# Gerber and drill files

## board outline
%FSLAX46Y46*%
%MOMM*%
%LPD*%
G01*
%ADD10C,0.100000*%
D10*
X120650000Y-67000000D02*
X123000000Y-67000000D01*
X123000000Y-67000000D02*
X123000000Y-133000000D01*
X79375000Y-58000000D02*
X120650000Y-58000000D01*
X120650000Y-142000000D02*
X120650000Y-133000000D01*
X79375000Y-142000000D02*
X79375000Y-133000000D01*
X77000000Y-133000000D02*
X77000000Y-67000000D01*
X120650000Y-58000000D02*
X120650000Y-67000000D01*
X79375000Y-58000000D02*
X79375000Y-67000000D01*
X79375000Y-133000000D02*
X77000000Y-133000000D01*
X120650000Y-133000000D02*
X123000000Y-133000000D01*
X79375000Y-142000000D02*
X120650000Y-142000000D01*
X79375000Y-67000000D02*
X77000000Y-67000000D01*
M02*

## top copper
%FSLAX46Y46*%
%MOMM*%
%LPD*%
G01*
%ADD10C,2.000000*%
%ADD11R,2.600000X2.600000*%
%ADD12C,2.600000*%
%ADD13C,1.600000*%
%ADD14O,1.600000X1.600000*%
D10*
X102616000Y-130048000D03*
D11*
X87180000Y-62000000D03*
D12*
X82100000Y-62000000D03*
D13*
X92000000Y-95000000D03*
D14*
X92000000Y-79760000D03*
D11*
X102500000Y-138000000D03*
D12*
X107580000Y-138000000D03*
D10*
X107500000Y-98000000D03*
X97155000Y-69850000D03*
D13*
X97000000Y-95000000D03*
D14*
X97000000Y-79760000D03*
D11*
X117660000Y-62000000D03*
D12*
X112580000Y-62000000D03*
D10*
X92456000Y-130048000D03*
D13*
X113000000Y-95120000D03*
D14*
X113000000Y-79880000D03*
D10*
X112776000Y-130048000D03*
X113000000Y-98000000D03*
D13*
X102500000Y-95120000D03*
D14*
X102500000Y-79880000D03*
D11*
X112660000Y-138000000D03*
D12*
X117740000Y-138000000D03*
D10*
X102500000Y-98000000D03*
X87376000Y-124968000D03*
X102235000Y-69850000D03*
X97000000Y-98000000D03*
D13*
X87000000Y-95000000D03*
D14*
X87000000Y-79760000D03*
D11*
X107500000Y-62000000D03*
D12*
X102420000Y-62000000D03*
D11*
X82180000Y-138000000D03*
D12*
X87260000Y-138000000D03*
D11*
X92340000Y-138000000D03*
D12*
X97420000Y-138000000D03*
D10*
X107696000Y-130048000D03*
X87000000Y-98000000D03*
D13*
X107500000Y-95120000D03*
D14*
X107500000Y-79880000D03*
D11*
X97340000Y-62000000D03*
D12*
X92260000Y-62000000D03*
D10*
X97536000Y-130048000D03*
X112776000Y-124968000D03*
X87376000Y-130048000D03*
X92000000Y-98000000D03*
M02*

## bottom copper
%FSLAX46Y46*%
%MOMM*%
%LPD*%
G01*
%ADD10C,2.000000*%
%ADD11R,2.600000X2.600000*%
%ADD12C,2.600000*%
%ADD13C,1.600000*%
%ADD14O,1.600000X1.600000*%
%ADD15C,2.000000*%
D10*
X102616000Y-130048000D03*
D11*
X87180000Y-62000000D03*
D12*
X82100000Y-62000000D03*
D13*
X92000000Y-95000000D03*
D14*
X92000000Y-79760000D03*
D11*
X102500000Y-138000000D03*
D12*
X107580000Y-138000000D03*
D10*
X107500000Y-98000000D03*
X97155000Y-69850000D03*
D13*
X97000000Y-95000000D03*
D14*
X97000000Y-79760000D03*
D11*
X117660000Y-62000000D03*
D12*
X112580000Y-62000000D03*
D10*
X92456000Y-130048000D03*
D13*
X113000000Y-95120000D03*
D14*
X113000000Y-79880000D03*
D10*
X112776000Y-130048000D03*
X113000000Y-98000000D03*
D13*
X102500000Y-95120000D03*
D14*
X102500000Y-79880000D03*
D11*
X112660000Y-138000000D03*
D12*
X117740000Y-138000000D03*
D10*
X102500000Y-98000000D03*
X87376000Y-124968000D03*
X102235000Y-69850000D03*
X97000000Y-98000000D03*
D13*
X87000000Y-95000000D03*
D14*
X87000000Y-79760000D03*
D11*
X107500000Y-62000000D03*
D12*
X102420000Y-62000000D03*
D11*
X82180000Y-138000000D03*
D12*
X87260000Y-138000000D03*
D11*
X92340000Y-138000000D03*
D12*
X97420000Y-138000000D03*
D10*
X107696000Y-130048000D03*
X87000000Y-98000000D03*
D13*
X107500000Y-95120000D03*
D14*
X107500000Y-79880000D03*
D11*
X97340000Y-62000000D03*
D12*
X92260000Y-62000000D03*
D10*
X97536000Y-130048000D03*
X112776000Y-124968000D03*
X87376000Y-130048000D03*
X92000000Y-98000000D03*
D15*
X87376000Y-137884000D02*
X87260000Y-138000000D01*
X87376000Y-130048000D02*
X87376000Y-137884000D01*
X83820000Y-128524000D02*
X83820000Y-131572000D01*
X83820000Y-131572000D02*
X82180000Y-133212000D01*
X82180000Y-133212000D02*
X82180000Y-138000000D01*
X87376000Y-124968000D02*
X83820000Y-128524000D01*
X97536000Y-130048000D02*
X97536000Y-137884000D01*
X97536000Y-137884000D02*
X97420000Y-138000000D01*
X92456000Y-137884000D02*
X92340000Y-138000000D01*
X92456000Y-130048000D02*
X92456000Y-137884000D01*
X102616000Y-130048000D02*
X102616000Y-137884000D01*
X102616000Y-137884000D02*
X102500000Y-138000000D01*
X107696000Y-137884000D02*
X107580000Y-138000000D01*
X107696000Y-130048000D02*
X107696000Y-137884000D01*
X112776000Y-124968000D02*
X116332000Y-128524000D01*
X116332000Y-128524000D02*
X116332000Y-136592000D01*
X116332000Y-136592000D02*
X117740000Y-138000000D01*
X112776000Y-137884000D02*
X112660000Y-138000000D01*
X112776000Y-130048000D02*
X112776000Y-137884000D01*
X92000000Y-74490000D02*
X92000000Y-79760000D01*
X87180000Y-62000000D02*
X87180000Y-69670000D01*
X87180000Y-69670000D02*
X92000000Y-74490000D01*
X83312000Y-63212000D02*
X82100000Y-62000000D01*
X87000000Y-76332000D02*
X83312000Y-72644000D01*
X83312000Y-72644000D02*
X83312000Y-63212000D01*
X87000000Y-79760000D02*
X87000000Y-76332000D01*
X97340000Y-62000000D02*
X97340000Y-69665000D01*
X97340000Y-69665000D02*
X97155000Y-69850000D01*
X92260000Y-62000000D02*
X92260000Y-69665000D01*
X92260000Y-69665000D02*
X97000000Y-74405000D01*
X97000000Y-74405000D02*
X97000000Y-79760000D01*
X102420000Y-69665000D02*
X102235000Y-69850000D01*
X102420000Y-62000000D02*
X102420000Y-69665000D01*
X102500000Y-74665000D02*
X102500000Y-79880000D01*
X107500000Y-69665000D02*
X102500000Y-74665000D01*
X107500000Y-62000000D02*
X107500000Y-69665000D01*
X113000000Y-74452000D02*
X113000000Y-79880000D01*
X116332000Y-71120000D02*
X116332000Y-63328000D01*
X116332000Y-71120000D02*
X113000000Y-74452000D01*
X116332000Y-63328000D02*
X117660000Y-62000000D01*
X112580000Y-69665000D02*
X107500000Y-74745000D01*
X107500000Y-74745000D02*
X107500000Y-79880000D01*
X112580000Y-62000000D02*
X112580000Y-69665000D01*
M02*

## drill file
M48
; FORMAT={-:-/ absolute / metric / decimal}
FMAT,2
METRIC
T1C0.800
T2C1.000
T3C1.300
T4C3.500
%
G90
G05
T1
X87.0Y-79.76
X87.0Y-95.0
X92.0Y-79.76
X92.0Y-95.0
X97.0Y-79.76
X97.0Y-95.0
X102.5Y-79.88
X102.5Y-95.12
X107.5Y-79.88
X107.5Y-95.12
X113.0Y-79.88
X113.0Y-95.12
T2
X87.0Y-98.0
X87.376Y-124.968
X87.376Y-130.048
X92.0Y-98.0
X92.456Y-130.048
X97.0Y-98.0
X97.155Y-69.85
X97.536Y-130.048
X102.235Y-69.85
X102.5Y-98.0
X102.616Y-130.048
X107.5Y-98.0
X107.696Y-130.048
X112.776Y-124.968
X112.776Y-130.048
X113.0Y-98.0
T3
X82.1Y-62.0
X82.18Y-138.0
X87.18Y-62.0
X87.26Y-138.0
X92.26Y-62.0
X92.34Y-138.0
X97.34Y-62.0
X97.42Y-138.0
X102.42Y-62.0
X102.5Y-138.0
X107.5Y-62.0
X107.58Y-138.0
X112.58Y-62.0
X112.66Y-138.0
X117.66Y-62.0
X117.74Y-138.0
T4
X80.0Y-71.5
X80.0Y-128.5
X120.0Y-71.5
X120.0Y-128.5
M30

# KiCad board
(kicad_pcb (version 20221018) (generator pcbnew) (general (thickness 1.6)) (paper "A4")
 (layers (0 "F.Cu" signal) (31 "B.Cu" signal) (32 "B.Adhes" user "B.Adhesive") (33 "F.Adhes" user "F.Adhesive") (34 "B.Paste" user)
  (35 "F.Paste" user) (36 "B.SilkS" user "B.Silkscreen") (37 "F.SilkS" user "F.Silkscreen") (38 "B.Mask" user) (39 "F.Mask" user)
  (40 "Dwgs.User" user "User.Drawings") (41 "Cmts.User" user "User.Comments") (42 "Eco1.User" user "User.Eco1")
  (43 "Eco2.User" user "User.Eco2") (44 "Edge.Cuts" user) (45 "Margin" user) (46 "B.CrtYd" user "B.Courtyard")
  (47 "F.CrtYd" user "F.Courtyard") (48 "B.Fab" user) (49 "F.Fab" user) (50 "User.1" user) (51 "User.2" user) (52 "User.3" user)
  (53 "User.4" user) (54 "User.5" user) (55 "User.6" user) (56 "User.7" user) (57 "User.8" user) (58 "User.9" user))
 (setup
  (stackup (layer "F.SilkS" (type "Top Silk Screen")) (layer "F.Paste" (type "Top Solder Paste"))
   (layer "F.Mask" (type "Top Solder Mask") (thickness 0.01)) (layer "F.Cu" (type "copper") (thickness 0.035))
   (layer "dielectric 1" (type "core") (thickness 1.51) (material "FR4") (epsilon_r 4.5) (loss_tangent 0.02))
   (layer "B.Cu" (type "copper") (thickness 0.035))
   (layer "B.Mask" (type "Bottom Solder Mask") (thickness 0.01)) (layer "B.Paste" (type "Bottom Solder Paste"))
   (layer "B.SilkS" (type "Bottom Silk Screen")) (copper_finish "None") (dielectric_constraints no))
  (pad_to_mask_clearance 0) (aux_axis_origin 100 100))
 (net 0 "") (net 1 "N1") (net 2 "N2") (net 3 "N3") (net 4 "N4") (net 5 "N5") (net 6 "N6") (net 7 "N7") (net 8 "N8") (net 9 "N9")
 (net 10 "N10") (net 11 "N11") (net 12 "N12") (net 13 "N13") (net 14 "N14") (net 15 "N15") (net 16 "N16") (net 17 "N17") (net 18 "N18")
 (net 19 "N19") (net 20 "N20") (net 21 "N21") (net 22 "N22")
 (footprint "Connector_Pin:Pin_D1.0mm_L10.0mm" (layer "F.Cu") (at 102.616 130.048)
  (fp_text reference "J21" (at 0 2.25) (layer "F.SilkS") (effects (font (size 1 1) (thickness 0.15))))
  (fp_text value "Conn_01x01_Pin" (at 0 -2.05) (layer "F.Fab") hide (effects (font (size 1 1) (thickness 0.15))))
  (pad "1" thru_hole circle (at 0 0) (size 2 2) (drill 1) (layers "*.Cu" "*.Mask") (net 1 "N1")))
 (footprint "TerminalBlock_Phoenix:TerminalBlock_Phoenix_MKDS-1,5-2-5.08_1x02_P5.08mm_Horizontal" (layer "F.Cu") (at 87.18 62 180)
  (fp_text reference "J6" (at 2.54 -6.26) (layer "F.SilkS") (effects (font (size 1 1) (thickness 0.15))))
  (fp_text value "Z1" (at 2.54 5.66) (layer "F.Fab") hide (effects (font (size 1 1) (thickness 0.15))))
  (pad "1" thru_hole rect (at 0 0 180) (size 2.6 2.6) (drill 1.3) (layers "*.Cu" "*.Mask") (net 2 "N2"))
  (pad "2" thru_hole circle (at 5.08 0 180) (size 2.6 2.6) (drill 1.3) (layers "*.Cu" "*.Mask") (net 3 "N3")))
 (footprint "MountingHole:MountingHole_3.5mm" (layer "F.Cu") (at 80 71.5)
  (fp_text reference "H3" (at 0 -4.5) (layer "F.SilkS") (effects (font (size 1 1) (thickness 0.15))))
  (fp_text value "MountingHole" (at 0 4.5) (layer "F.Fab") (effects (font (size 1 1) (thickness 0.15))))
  (pad "" np_thru_hole circle (at 0 0) (size 3.5 3.5) (drill 3.5) (layers "*.Cu" "*.Mask")))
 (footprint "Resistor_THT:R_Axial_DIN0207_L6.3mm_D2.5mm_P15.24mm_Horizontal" (layer "F.Cu") (at 92 95 90)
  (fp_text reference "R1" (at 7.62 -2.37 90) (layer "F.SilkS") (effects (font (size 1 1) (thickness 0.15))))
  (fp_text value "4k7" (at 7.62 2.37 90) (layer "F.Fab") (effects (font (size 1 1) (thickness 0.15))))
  (pad "1" thru_hole circle (at 0 0 90) (size 1.6 1.6) (drill 0.8) (layers "*.Cu" "*.Mask") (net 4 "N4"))
  (pad "2" thru_hole oval (at 15.24 0 90) (size 1.6 1.6) (drill 0.8) (layers "*.Cu" "*.Mask") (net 2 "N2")))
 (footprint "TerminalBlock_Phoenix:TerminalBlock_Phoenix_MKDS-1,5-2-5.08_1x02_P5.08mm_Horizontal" (layer "F.Cu") (at 102.5 138)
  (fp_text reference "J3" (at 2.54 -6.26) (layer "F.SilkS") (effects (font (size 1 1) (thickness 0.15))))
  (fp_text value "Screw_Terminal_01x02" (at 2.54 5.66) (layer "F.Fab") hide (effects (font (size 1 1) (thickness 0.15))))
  (pad "1" thru_hole rect (at 0 0) (size 2.6 2.6) (drill 1.3) (layers "*.Cu" "*.Mask") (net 1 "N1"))
  (pad "2" thru_hole circle (at 5.08 0) (size 2.6 2.6) (drill 1.3) (layers "*.Cu" "*.Mask") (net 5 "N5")))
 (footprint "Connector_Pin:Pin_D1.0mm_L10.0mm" (layer "F.Cu") (at 107.5 98)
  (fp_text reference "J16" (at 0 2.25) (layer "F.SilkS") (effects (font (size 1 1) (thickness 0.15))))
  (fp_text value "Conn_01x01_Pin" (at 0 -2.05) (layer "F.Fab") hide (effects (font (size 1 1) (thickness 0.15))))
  (pad "1" thru_hole circle (at 0 0) (size 2 2) (drill 1) (layers "*.Cu" "*.Mask") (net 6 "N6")))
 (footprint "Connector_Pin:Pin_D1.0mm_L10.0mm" (layer "F.Cu") (at 97.155 69.85)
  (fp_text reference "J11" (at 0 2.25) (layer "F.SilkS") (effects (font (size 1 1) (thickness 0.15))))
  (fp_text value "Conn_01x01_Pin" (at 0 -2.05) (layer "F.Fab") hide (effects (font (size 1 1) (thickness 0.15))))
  (pad "1" thru_hole circle (at 0 0) (size 2 2) (drill 1) (layers "*.Cu" "*.Mask") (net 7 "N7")))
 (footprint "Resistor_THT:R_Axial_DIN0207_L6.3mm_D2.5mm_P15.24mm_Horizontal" (layer "F.Cu") (at 97 95 90)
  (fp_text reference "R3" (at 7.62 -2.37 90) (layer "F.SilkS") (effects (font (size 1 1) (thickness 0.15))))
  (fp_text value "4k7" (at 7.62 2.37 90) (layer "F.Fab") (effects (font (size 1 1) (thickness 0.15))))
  (pad "1" thru_hole circle (at 0 0 90) (size 1.6 1.6) (drill 0.8) (layers "*.Cu" "*.Mask") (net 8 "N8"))
  (pad "2" thru_hole oval (at 15.24 0 90) (size 1.6 1.6) (drill 0.8) (layers "*.Cu" "*.Mask") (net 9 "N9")))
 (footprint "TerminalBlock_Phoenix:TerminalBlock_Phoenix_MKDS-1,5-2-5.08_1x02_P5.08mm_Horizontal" (layer "F.Cu") (at 117.66 62 180)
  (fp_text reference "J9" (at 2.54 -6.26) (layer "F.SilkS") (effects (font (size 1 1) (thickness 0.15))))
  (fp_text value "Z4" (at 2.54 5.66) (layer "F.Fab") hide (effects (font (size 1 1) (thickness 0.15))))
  (pad "1" thru_hole rect (at 0 0 180) (size 2.6 2.6) (drill 1.3) (layers "*.Cu" "*.Mask") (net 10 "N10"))
  (pad "2" thru_hole circle (at 5.08 0 180) (size 2.6 2.6) (drill 1.3) (layers "*.Cu" "*.Mask") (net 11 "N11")))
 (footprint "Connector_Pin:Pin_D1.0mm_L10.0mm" (layer "F.Cu") (at 92.456 130.048)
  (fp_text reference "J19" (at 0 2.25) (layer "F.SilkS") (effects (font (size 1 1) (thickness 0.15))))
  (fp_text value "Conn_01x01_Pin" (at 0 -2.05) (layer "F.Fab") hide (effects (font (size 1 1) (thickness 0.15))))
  (pad "1" thru_hole circle (at 0 0) (size 2 2) (drill 1) (layers "*.Cu" "*.Mask") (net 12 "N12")))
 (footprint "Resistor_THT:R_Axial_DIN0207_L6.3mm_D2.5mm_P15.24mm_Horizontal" (layer "F.Cu") (at 113 95.12 90)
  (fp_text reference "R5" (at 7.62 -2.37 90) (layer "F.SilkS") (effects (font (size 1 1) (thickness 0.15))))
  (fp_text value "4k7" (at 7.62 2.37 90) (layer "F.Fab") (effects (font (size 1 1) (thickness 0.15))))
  (pad "1" thru_hole circle (at 0 0 90) (size 1.6 1.6) (drill 0.8) (layers "*.Cu" "*.Mask") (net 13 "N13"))
  (pad "2" thru_hole oval (at 15.24 0 90) (size 1.6 1.6) (drill 0.8) (layers "*.Cu" "*.Mask") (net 10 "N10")))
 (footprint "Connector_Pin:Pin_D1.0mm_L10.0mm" (layer "F.Cu") (at 112.776 130.048)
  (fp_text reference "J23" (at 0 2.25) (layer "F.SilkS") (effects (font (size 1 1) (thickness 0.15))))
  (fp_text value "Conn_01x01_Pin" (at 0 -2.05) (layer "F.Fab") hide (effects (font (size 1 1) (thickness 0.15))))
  (pad "1" thru_hole circle (at 0 0) (size 2 2) (drill 1) (layers "*.Cu" "*.Mask") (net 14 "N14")))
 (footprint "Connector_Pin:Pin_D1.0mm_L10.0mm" (layer "F.Cu") (at 113 98)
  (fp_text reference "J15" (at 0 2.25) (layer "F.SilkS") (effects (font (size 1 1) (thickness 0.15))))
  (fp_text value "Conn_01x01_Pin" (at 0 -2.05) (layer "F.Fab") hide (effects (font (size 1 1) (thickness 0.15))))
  (pad "1" thru_hole circle (at 0 0) (size 2 2) (drill 1) (layers "*.Cu" "*.Mask") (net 13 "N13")))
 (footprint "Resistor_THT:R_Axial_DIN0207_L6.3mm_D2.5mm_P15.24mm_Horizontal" (layer "F.Cu") (at 102.5 95.12 90)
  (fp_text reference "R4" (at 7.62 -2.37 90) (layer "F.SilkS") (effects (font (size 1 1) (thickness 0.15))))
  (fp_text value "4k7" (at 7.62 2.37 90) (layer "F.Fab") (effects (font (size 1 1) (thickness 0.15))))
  (pad "1" thru_hole circle (at 0 0 90) (size 1.6 1.6) (drill 0.8) (layers "*.Cu" "*.Mask") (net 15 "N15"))
  (pad "2" thru_hole oval (at 15.24 0 90) (size 1.6 1.6) (drill 0.8) (layers "*.Cu" "*.Mask") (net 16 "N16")))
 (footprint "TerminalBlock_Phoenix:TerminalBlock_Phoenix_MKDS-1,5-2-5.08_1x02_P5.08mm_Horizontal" (layer "F.Cu") (at 112.66 138)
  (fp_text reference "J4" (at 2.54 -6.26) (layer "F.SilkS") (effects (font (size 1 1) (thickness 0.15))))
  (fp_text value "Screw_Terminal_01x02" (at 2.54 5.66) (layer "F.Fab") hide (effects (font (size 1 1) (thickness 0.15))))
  (pad "1" thru_hole rect (at 0 0) (size 2.6 2.6) (drill 1.3) (layers "*.Cu" "*.Mask") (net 14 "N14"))
  (pad "2" thru_hole circle (at 5.08 0) (size 2.6 2.6) (drill 1.3) (layers "*.Cu" "*.Mask") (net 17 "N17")))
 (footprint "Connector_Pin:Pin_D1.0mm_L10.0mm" (layer "F.Cu") (at 102.5 98)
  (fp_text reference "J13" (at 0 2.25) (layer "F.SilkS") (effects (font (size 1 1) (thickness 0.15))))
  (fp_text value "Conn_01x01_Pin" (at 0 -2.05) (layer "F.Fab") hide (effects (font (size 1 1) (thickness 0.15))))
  (pad "1" thru_hole circle (at 0 0) (size 2 2) (drill 1) (layers "*.Cu" "*.Mask") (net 15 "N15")))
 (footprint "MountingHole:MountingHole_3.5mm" (layer "F.Cu") (at 120 128.5)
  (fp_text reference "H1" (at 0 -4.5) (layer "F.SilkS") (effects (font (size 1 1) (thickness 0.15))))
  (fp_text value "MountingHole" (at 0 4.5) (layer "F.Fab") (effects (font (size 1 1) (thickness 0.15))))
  (pad "" np_thru_hole circle (at 0 0) (size 3.5 3.5) (drill 3.5) (layers "*.Cu" "*.Mask")))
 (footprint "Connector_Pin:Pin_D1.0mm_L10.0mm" (layer "F.Cu") (at 87.376 124.968)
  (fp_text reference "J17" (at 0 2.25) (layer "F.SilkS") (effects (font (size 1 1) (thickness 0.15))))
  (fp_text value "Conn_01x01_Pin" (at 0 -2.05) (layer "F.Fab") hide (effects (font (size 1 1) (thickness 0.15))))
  (pad "1" thru_hole circle (at 0 0) (size 2 2) (drill 1) (layers "*.Cu" "*.Mask") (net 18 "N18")))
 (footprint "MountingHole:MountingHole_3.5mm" (layer "F.Cu") (at 80 128.5)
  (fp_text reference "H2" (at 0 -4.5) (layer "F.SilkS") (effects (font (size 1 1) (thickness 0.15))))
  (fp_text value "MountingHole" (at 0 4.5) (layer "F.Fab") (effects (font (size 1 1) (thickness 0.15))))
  (pad "" np_thru_hole circle (at 0 0) (size 3.5 3.5) (drill 3.5) (layers "*.Cu" "*.Mask")))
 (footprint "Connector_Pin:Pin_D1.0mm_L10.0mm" (layer "F.Cu") (at 102.235 69.85)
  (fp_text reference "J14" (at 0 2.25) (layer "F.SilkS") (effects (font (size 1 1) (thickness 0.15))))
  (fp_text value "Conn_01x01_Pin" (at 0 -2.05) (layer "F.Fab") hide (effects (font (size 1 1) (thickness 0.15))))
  (pad "1" thru_hole circle (at 0 0) (size 2 2) (drill 1) (layers "*.Cu" "*.Mask") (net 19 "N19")))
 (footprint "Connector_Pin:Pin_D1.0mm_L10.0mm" (layer "F.Cu") (at 97 98)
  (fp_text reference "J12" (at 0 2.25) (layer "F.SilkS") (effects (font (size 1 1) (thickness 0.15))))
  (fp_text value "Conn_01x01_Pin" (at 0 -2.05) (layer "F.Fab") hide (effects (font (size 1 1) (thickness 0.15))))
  (pad "1" thru_hole circle (at 0 0) (size 2 2) (drill 1) (layers "*.Cu" "*.Mask") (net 8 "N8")))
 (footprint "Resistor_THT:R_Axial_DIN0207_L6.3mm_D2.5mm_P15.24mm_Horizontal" (layer "F.Cu") (at 87 95 90)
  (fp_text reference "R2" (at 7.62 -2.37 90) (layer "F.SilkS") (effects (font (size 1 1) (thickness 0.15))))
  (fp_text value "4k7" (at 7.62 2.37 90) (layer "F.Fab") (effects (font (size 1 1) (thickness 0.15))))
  (pad "1" thru_hole circle (at 0 0 90) (size 1.6 1.6) (drill 0.8) (layers "*.Cu" "*.Mask") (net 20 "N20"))
  (pad "2" thru_hole oval (at 15.24 0 90) (size 1.6 1.6) (drill 0.8) (layers "*.Cu" "*.Mask") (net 3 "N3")))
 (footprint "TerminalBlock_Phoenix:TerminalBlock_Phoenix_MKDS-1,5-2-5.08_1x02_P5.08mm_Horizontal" (layer "F.Cu") (at 107.5 62 180)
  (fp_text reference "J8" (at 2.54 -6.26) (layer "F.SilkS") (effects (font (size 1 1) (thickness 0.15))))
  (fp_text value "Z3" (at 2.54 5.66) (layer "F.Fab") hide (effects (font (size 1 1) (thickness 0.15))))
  (pad "1" thru_hole rect (at 0 0 180) (size 2.6 2.6) (drill 1.3) (layers "*.Cu" "*.Mask") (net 16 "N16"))
  (pad "2" thru_hole circle (at 5.08 0 180) (size 2.6 2.6) (drill 1.3) (layers "*.Cu" "*.Mask") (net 19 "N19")))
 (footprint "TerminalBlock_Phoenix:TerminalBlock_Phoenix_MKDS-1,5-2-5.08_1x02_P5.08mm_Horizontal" (layer "F.Cu") (at 82.18 138)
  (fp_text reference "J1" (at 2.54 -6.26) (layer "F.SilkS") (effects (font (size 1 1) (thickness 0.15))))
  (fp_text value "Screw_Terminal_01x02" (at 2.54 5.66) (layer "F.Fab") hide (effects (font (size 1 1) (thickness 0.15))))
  (pad "1" thru_hole rect (at 0 0) (size 2.6 2.6) (drill 1.3) (layers "*.Cu" "*.Mask") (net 18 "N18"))
  (pad "2" thru_hole circle (at 5.08 0) (size 2.6 2.6) (drill 1.3) (layers "*.Cu" "*.Mask") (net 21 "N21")))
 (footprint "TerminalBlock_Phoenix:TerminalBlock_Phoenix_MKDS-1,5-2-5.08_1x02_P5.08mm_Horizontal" (layer "F.Cu") (at 92.34 138)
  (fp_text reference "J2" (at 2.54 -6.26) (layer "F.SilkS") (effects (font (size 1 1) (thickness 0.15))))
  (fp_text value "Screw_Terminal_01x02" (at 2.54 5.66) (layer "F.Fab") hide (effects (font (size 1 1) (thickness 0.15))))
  (pad "1" thru_hole rect (at 0 0) (size 2.6 2.6) (drill 1.3) (layers "*.Cu" "*.Mask") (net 12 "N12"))
  (pad "2" thru_hole circle (at 5.08 0) (size 2.6 2.6) (drill 1.3) (layers "*.Cu" "*.Mask") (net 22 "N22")))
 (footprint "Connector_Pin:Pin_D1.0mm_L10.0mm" (layer "F.Cu") (at 107.696 130.048)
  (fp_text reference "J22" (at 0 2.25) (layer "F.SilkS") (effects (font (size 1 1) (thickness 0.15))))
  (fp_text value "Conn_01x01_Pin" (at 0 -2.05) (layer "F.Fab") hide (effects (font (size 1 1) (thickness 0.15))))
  (pad "1" thru_hole circle (at 0 0) (size 2 2) (drill 1) (layers "*.Cu" "*.Mask") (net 5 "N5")))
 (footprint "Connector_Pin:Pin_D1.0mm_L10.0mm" (layer "F.Cu") (at 87 98)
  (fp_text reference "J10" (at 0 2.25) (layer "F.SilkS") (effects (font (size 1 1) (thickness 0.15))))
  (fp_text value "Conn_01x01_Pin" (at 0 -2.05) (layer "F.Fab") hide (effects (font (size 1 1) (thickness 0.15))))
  (pad "1" thru_hole circle (at 0 0) (size 2 2) (drill 1) (layers "*.Cu" "*.Mask") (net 20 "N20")))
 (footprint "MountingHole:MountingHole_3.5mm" (layer "F.Cu") (at 120 71.5)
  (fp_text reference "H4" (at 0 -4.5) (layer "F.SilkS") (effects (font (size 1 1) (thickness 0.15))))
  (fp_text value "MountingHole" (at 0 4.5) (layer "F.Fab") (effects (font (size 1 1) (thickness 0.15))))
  (pad "" np_thru_hole circle (at 0 0) (size 3.5 3.5) (drill 3.5) (layers "*.Cu" "*.Mask")))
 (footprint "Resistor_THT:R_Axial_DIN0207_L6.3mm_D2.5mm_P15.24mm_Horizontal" (layer "F.Cu") (at 107.5 95.12 90)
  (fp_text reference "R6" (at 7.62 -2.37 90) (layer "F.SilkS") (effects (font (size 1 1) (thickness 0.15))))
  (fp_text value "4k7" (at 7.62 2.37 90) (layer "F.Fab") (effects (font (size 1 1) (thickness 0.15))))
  (pad "1" thru_hole circle (at 0 0 90) (size 1.6 1.6) (drill 0.8) (layers "*.Cu" "*.Mask") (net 6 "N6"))
  (pad "2" thru_hole oval (at 15.24 0 90) (size 1.6 1.6) (drill 0.8) (layers "*.Cu" "*.Mask") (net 11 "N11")))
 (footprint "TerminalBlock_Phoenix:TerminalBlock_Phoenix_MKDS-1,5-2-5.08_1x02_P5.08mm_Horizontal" (layer "F.Cu") (at 97.34 62 180)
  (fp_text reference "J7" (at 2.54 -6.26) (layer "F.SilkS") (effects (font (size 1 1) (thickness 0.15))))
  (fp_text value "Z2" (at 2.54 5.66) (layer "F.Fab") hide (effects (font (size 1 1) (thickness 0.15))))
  (pad "1" thru_hole rect (at 0 0 180) (size 2.6 2.6) (drill 1.3) (layers "*.Cu" "*.Mask") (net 7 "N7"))
  (pad "2" thru_hole circle (at 5.08 0 180) (size 2.6 2.6) (drill 1.3) (layers "*.Cu" "*.Mask") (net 9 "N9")))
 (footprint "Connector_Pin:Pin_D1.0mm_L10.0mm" (layer "F.Cu") (at 97.536 130.048)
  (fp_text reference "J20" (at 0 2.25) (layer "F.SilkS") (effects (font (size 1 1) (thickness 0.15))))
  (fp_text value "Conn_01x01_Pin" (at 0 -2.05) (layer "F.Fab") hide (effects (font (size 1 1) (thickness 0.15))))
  (pad "1" thru_hole circle (at 0 0) (size 2 2) (drill 1) (layers "*.Cu" "*.Mask") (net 22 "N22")))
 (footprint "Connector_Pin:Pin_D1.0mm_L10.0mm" (layer "F.Cu") (at 112.776 124.968)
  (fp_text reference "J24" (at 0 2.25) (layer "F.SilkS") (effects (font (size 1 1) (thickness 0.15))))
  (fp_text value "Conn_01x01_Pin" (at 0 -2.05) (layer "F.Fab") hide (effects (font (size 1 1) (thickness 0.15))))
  (pad "1" thru_hole circle (at 0 0) (size 2 2) (drill 1) (layers "*.Cu" "*.Mask") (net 17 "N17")))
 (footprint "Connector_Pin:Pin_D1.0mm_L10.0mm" (layer "F.Cu") (at 87.376 130.048)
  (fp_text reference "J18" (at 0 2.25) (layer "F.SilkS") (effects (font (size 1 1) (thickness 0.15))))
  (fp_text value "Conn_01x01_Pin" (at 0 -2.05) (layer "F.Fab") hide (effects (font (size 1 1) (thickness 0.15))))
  (pad "1" thru_hole circle (at 0 0) (size 2 2) (drill 1) (layers "*.Cu" "*.Mask") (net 21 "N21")))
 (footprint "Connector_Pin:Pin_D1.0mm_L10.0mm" (layer "F.Cu") (at 92 98)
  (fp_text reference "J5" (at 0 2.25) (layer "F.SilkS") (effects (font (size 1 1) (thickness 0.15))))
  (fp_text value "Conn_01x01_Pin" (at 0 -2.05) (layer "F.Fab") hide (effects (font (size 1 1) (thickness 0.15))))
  (pad "1" thru_hole circle (at 0 0) (size 2 2) (drill 1) (layers "*.Cu" "*.Mask") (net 4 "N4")))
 (gr_line (start 120.65 67) (end 123 67) (stroke (width 0.1) (type solid)) (layer "Edge.Cuts"))
 (gr_line (start 123 67) (end 123 133) (stroke (width 0.1) (type solid)) (layer "Edge.Cuts"))
 (gr_line (start 79.375 58) (end 120.65 58) (stroke (width 0.1) (type solid)) (layer "Edge.Cuts"))
 (gr_line (start 120.65 142) (end 120.65 133) (stroke (width 0.1) (type solid)) (layer "Edge.Cuts"))
 (gr_line (start 79.375 142) (end 79.375 133) (stroke (width 0.1) (type solid)) (layer "Edge.Cuts"))
 (gr_line (start 77 133) (end 77 67) (stroke (width 0.1) (type solid)) (layer "Edge.Cuts"))
 (gr_line (start 120.65 58) (end 120.65 67) (stroke (width 0.1) (type solid)) (layer "Edge.Cuts"))
 (gr_line (start 79.375 58) (end 79.375 67) (stroke (width 0.1) (type solid)) (layer "Edge.Cuts"))
 (gr_line (start 79.375 133) (end 77 133) (stroke (width 0.1) (type solid)) (layer "Edge.Cuts"))
 (gr_line (start 120.65 133) (end 123 133) (stroke (width 0.1) (type solid)) (layer "Edge.Cuts"))
 (gr_line (start 79.375 142) (end 120.65 142) (stroke (width 0.1) (type solid)) (layer "Edge.Cuts"))
 (gr_line (start 79.375 67) (end 77 67) (stroke (width 0.1) (type solid)) (layer "Edge.Cuts"))
 (segment (start 87.376 137.884) (end 87.26 138) (width 2) (layer "B.Cu") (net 21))
 (segment (start 87.376 130.048) (end 87.376 137.884) (width 2) (layer "B.Cu") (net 21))
 (segment (start 83.82 128.524) (end 83.82 131.572) (width 2) (layer "B.Cu") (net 18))
 (segment (start 83.82 131.572) (end 82.18 133.212) (width 2) (layer "B.Cu") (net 18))
 (segment (start 82.18 133.212) (end 82.18 138) (width 2) (layer "B.Cu") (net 18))
 (segment (start 87.376 124.968) (end 83.82 128.524) (width 2) (layer "B.Cu") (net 18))
 (segment (start 97.536 130.048) (end 97.536 137.884) (width 2) (layer "B.Cu") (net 22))
 (segment (start 97.536 137.884) (end 97.42 138) (width 2) (layer "B.Cu") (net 22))
 (segment (start 92.456 137.884) (end 92.34 138) (width 2) (layer "B.Cu") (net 12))
 (segment (start 92.456 130.048) (end 92.456 137.884) (width 2) (layer "B.Cu") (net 12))
 (segment (start 102.616 130.048) (end 102.616 137.884) (width 2) (layer "B.Cu") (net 1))
 (segment (start 102.616 137.884) (end 102.5 138) (width 2) (layer "B.Cu") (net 1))
 (segment (start 107.696 137.884) (end 107.58 138) (width 2) (layer "B.Cu") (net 5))
 (segment (start 107.696 130.048) (end 107.696 137.884) (width 2) (layer "B.Cu") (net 5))
 (segment (start 112.776 124.968) (end 116.332 128.524) (width 2) (layer "B.Cu") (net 17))
 (segment (start 116.332 128.524) (end 116.332 136.592) (width 2) (layer "B.Cu") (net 17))
 (segment (start 116.332 136.592) (end 117.74 138) (width 2) (layer "B.Cu") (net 17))
 (segment (start 112.776 137.884) (end 112.66 138) (width 2) (layer "B.Cu") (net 14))
 (segment (start 112.776 130.048) (end 112.776 137.884) (width 2) (layer "B.Cu") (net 14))
 (segment (start 92 74.49) (end 92 79.76) (width 2) (layer "B.Cu") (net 2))
 (segment (start 87.18 62) (end 87.18 69.67) (width 2) (layer "B.Cu") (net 2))
 (segment (start 87.18 69.67) (end 92 74.49) (width 2) (layer "B.Cu") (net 2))
 (segment (start 83.312 63.212) (end 82.1 62) (width 2) (layer "B.Cu") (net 3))
 (segment (start 87 76.332) (end 83.312 72.644) (width 2) (layer "B.Cu") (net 3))
 (segment (start 83.312 72.644) (end 83.312 63.212) (width 2) (layer "B.Cu") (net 3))
 (segment (start 87 79.76) (end 87 76.332) (width 2) (layer "B.Cu") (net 3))
 (segment (start 97.34 62) (end 97.34 69.665) (width 2) (layer "B.Cu") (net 7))
 (segment (start 97.34 69.665) (end 97.155 69.85) (width 2) (layer "B.Cu") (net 7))
 (segment (start 92.26 62) (end 92.26 69.665) (width 2) (layer "B.Cu") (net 9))
 (segment (start 92.26 69.665) (end 97 74.405) (width 2) (layer "B.Cu") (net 9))
 (segment (start 97 74.405) (end 97 79.76) (width 2) (layer "B.Cu") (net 9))
 (segment (start 102.42 69.665) (end 102.235 69.85) (width 2) (layer "B.Cu") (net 19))
 (segment (start 102.42 62) (end 102.42 69.665) (width 2) (layer "B.Cu") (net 19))
 (segment (start 102.5 74.665) (end 102.5 79.88) (width 2) (layer "B.Cu") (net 16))
 (segment (start 107.5 69.665) (end 102.5 74.665) (width 2) (layer "B.Cu") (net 16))
 (segment (start 107.5 62) (end 107.5 69.665) (width 2) (layer "B.Cu") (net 16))
 (segment (start 113 74.452) (end 113 79.88) (width 2) (layer "B.Cu") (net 10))
 (segment (start 116.332 71.12) (end 116.332 63.328) (width 2) (layer "B.Cu") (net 10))
 (segment (start 116.332 71.12) (end 113 74.452) (width 2) (layer "B.Cu") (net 10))
 (segment (start 116.332 63.328) (end 117.66 62) (width 2) (layer "B.Cu") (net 10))
 (segment (start 112.58 69.665) (end 107.5 74.745) (width 2) (layer "B.Cu") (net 11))
 (segment (start 107.5 74.745) (end 107.5 79.88) (width 2) (layer "B.Cu") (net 11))
 (segment (start 112.58 62) (end 112.58 69.665) (width 2) (layer "B.Cu") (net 11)))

